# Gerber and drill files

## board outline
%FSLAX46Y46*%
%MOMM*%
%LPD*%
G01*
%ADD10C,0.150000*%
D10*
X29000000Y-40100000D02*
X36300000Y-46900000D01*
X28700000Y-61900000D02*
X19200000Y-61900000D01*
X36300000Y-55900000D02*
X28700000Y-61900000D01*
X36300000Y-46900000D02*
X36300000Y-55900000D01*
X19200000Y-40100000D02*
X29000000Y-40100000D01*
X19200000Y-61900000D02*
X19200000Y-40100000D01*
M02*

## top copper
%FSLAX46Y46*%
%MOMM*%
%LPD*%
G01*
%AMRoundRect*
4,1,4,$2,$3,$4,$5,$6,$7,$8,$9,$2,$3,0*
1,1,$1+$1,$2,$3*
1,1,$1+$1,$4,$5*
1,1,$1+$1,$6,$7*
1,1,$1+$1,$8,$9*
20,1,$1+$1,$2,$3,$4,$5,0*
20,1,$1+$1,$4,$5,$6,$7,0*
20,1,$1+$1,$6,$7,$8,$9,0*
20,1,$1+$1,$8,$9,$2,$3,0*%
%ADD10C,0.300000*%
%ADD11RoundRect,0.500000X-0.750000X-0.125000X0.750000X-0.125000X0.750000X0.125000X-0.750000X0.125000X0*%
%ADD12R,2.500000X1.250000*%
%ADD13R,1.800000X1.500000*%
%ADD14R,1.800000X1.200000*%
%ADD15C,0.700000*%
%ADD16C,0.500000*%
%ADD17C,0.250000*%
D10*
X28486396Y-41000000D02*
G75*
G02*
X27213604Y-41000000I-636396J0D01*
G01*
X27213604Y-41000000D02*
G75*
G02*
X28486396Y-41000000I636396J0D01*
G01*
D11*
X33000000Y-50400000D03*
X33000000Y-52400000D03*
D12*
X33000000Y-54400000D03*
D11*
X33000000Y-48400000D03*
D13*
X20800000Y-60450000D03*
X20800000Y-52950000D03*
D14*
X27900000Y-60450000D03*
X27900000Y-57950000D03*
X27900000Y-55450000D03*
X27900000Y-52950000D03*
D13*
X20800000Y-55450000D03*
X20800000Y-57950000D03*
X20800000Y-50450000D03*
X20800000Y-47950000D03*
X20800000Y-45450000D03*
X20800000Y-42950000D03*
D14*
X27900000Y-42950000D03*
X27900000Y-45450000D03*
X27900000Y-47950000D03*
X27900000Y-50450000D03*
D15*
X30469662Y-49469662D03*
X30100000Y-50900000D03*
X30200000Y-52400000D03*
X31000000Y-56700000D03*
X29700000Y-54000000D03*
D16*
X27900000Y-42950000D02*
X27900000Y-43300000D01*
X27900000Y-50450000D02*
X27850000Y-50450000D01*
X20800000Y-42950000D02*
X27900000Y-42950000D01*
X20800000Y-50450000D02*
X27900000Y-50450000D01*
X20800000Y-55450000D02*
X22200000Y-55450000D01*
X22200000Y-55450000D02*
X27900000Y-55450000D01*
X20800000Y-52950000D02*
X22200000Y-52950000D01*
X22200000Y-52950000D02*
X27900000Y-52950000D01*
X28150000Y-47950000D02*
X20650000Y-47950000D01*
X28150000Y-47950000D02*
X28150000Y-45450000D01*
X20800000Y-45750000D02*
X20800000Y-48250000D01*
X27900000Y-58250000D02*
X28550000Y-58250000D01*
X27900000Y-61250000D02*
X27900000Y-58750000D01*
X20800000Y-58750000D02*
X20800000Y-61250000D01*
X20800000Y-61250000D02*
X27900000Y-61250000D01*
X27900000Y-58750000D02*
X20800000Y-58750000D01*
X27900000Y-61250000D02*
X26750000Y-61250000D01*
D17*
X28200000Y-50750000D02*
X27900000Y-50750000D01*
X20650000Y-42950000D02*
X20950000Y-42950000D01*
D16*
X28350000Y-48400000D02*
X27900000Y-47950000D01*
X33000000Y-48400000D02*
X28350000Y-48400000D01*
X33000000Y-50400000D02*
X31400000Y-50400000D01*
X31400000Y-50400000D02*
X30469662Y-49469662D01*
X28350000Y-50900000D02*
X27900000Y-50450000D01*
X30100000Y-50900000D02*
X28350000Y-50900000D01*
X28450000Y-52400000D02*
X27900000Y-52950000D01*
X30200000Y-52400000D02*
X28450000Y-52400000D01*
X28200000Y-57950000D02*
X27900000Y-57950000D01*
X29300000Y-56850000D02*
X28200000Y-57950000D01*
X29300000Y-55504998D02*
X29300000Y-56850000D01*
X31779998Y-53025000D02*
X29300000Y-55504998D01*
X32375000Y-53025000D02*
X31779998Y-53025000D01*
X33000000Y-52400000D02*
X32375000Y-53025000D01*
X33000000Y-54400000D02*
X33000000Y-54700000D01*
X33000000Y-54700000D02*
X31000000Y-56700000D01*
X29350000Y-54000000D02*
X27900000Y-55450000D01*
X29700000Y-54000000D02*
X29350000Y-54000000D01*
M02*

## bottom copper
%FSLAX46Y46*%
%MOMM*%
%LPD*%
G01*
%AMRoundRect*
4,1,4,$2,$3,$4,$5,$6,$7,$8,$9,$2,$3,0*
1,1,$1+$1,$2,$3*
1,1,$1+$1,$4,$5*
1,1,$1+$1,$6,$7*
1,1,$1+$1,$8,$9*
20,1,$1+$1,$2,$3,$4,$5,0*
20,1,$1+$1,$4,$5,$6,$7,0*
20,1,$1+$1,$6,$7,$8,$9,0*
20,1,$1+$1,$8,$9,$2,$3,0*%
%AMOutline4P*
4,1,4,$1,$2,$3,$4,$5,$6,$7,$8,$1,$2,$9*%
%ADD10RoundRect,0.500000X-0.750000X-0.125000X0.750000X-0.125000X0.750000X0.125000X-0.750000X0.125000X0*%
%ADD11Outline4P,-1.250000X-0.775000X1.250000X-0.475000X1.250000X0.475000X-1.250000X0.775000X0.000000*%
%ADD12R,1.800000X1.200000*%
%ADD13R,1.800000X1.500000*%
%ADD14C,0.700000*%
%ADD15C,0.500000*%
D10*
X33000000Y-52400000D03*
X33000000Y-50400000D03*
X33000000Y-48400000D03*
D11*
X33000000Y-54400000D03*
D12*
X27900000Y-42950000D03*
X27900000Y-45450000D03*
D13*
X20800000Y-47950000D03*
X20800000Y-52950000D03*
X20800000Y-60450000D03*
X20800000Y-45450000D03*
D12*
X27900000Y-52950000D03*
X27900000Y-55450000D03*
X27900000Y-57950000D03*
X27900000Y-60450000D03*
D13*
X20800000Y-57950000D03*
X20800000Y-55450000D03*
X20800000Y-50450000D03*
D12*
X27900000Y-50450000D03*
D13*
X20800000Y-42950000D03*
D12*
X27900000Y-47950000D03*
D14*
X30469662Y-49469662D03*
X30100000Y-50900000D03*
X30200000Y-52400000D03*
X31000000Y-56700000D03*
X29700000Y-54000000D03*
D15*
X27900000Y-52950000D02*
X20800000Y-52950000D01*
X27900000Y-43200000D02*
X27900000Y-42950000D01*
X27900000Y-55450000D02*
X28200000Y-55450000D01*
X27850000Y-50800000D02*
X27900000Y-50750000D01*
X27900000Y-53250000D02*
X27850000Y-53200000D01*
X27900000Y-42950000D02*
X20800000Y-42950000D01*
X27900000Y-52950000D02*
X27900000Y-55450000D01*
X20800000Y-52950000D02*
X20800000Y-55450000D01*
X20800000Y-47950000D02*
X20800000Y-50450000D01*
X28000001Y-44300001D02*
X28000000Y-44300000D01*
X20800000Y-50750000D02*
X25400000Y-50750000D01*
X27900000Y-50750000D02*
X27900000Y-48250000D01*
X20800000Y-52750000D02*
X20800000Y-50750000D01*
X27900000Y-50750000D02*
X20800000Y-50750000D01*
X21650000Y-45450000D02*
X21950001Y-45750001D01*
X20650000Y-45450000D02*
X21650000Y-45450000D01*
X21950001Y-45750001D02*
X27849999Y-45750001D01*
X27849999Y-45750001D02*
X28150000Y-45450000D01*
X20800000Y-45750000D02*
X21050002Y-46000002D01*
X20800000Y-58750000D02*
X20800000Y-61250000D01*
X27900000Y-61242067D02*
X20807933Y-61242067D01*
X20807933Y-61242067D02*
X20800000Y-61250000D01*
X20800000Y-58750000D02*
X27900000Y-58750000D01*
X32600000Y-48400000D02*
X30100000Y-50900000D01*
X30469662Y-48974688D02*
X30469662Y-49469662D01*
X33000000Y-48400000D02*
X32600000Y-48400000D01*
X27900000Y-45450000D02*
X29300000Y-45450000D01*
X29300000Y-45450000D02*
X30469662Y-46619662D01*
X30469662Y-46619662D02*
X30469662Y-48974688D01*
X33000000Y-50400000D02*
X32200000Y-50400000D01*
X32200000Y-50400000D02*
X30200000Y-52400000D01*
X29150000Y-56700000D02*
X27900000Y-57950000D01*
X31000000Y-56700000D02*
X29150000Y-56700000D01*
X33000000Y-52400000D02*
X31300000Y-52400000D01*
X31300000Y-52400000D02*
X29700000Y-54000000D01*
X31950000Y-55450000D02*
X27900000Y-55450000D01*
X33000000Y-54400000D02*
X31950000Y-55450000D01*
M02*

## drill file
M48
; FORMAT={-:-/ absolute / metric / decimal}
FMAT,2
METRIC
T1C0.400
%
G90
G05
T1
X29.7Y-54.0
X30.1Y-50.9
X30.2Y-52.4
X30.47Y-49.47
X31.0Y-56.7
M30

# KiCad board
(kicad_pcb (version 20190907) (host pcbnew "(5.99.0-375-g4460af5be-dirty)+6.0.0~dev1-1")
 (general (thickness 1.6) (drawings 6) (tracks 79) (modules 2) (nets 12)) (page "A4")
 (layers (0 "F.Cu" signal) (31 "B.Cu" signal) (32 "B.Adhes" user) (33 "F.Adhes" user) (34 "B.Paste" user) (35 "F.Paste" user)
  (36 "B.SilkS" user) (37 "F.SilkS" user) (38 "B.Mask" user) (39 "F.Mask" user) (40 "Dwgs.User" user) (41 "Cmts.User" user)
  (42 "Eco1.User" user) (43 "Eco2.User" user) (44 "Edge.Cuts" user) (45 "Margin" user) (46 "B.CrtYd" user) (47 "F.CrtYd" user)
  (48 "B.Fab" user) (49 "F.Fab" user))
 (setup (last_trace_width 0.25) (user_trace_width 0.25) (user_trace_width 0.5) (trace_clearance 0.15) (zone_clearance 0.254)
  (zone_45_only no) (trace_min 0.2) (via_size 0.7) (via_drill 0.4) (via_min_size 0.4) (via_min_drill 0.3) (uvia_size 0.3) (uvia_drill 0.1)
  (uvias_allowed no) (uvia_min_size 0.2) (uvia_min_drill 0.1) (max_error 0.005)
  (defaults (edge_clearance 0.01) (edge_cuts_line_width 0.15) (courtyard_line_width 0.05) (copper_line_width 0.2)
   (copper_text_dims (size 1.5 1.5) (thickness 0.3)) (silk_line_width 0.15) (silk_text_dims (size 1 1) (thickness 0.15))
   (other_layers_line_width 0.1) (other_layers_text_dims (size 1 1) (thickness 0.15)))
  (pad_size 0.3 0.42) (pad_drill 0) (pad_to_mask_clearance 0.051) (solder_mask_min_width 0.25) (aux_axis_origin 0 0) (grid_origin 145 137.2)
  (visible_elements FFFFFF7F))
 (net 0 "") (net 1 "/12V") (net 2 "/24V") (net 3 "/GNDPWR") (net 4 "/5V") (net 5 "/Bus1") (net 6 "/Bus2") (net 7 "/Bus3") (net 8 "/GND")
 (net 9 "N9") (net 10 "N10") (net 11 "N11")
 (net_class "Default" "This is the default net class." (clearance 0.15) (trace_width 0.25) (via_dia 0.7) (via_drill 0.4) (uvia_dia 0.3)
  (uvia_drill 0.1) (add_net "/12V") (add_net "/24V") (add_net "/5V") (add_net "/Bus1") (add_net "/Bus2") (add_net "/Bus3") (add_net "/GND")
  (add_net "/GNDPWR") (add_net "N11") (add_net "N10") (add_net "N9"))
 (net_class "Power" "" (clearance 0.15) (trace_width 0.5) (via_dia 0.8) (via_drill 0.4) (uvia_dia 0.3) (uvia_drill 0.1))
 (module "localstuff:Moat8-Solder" (layer "B.Cu") (at 33 55.9)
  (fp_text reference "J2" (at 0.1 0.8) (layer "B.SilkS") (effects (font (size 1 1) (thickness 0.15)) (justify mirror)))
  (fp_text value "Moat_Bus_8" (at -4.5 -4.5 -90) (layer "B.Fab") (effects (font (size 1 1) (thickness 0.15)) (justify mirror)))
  (pad "6" smd roundrect (at 0 -5.5) (size 2.5 1.25) (layers "F.Cu" "F.Mask") (roundrect_rratio 0.4) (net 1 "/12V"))
  (pad "7" smd roundrect (at 0 -3.5) (size 2.5 1.25) (layers "F.Cu" "F.Mask") (roundrect_rratio 0.4) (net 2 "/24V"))
  (pad "8" smd rect (at 0 -1.5) (size 2.5 1.25) (layers "F.Cu" "F.Mask") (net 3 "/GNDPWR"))
  (pad "5" smd roundrect (at 0 -7.5) (size 2.5 1.25) (layers "F.Cu" "F.Mask") (roundrect_rratio 0.4) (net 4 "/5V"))
  (pad "2" smd roundrect (at 0 -3.5) (size 2.5 1.25) (layers "B.Cu" "B.Mask") (roundrect_rratio 0.4) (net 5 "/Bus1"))
  (pad "3" smd roundrect (at 0 -5.5) (size 2.5 1.25) (layers "B.Cu" "B.Mask") (roundrect_rratio 0.4) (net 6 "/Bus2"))
  (pad "4" smd roundrect (at 0 -7.5) (size 2.5 1.25) (layers "B.Cu" "B.Mask") (roundrect_rratio 0.4) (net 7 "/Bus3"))
  (pad "1" smd trapezoid (at 0 -1.5) (size 2.5 1.25) (rect_delta 0.3 0) (layers "B.Cu" "B.Mask") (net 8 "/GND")))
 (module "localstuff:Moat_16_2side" (layer "F.Cu") (at 24.4 52 -90)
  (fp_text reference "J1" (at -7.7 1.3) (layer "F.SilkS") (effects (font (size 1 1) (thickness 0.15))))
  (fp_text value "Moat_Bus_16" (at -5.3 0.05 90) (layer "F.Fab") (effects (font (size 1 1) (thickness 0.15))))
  (fp_circle (center -11 -3.45) (end -10.363604 -3.45) (layer "F.Cu") (width 0.3))
  (pad "2" smd rect (at -9.05 -3.5 90) (size 1.2 1.8) (layers "B.Cu" "B.Paste" "B.Mask") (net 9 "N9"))
  (pad "4" smd rect (at -6.55 -3.5 90) (size 1.2 1.8) (layers "B.Cu" "B.Paste" "B.Mask") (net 1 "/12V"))
  (pad "6" smd rect (at -4.05 3.6 90) (size 1.5 1.8) (layers "B.Cu" "B.Paste" "B.Mask") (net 8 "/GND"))
  (pad "10" smd rect (at 0.95 3.6 90) (size 1.5 1.8) (layers "B.Cu" "B.Paste" "B.Mask") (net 8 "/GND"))
  (pad "16" smd rect (at 8.45 3.6 90) (size 1.5 1.8) (layers "B.Cu" "B.Paste" "B.Mask") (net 3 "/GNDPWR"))
  (pad "4" smd rect (at -6.55 3.6 90) (size 1.5 1.8) (layers "B.Cu" "B.Paste" "B.Mask") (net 1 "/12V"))
  (pad "10" smd rect (at 0.95 -3.5 90) (size 1.2 1.8) (layers "B.Cu" "B.Paste" "B.Mask") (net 8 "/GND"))
  (pad "12" smd rect (at 3.45 -3.5 90) (size 1.2 1.8) (layers "B.Cu" "B.Paste" "B.Mask") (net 8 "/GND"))
  (pad "14" smd rect (at 5.95 -3.5 90) (size 1.2 1.8) (layers "B.Cu" "B.Paste" "B.Mask") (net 3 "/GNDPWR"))
  (pad "16" smd rect (at 8.45 -3.5 90) (size 1.2 1.8) (layers "B.Cu" "B.Paste" "B.Mask") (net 3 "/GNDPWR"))
  (pad "14" smd rect (at 5.95 3.6 90) (size 1.5 1.8) (layers "B.Cu" "B.Paste" "B.Mask") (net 3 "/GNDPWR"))
  (pad "12" smd rect (at 3.45 3.6 90) (size 1.5 1.8) (layers "B.Cu" "B.Paste" "B.Mask") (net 8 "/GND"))
  (pad "8" smd rect (at -1.55 3.6 90) (size 1.5 1.8) (layers "B.Cu" "B.Paste" "B.Mask") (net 8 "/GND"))
  (pad "8" smd rect (at -1.55 -3.5 90) (size 1.2 1.8) (layers "B.Cu" "B.Paste" "B.Mask") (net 8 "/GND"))
  (pad "2" smd rect (at -9.05 3.6 90) (size 1.5 1.8) (layers "B.Cu" "B.Paste" "B.Mask") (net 9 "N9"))
  (pad "6" smd rect (at -4.05 -3.5 90) (size 1.2 1.8) (layers "B.Cu" "B.Paste" "B.Mask") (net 8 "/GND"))
  (pad "15" smd rect (at 8.45 3.6 270) (size 1.5 1.8) (layers "F.Cu" "F.Paste" "F.Mask") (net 2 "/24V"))
  (pad "9" smd rect (at 0.95 3.6 270) (size 1.5 1.8) (layers "F.Cu" "F.Paste" "F.Mask") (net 6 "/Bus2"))
  (pad "15" smd rect (at 8.45 -3.5 270) (size 1.2 1.8) (layers "F.Cu" "F.Paste" "F.Mask") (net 2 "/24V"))
  (pad "13" smd rect (at 5.95 -3.5 270) (size 1.2 1.8) (layers "F.Cu" "F.Paste" "F.Mask") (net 2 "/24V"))
  (pad "11" smd rect (at 3.45 -3.5 270) (size 1.2 1.8) (layers "F.Cu" "F.Paste" "F.Mask") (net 5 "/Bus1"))
  (pad "9" smd rect (at 0.95 -3.5 270) (size 1.2 1.8) (layers "F.Cu" "F.Paste" "F.Mask") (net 6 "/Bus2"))
  (pad "11" smd rect (at 3.45 3.6 270) (size 1.5 1.8) (layers "F.Cu" "F.Paste" "F.Mask") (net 5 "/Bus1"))
  (pad "13" smd rect (at 5.95 3.6 270) (size 1.5 1.8) (layers "F.Cu" "F.Paste" "F.Mask") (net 2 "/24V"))
  (pad "7" smd rect (at -1.55 3.6 270) (size 1.5 1.8) (layers "F.Cu" "F.Paste" "F.Mask") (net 7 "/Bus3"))
  (pad "5" smd rect (at -4.05 3.6 270) (size 1.5 1.8) (layers "F.Cu" "F.Paste" "F.Mask") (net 4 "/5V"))
  (pad "3" smd rect (at -6.55 3.6 270) (size 1.5 1.8) (layers "F.Cu" "F.Paste" "F.Mask") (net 4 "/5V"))
  (pad "1" smd rect (at -9.05 3.6 270) (size 1.5 1.8) (layers "F.Cu" "F.Paste" "F.Mask") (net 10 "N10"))
  (pad "1" smd rect (at -9.05 -3.5 270) (size 1.2 1.8) (layers "F.Cu" "F.Paste" "F.Mask") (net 10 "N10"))
  (pad "3" smd rect (at -6.55 -3.5 270) (size 1.2 1.8) (layers "F.Cu" "F.Paste" "F.Mask") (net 4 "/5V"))
  (pad "5" smd rect (at -4.05 -3.5 270) (size 1.2 1.8) (layers "F.Cu" "F.Paste" "F.Mask") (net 4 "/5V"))
  (pad "7" smd rect (at -1.55 -3.5 270) (size 1.2 1.8) (layers "F.Cu" "F.Paste" "F.Mask") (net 7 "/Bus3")))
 (gr_line (start 29 40.1) (end 36.3 46.9) (layer "Edge.Cuts") (width 0.15))
 (gr_line (start 28.7 61.9) (end 19.2 61.9) (layer "Edge.Cuts") (width 0.15))
 (gr_line (start 36.3 55.9) (end 28.7 61.9) (layer "Edge.Cuts") (width 0.15))
 (gr_line (start 36.3 46.9) (end 36.3 55.9) (layer "Edge.Cuts") (width 0.15))
 (gr_line (start 19.2 40.1) (end 29 40.1) (layer "Edge.Cuts") (width 0.15))
 (gr_line (start 19.2 61.9) (end 19.2 40.1) (layer "Edge.Cuts") (width 0.15))
 (segment (start 27.9 52.95) (end 20.8 52.95) (width 0.5) (layer "B.Cu") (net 8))
 (segment (start 27.9 42.95) (end 27.9 43.3) (width 0.5) (layer "F.Cu") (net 10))
 (segment (start 27.9 43.2) (end 27.9 42.95) (width 0.5) (layer "B.Cu") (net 9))
 (segment (start 27.9 55.45) (end 28.2 55.45) (width 0.5) (layer "B.Cu") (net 8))
 (segment (start 27.85 50.8) (end 27.9 50.75) (width 0.5) (layer "B.Cu") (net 8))
 (segment (start 27.9 53.25) (end 27.85 53.2) (width 0.5) (layer "B.Cu") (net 8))
 (segment (start 27.9 50.45) (end 27.85 50.45) (width 0.5) (layer "F.Cu") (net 7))
 (segment (start 20.8 42.95) (end 27.9 42.95) (width 0.5) (layer "F.Cu") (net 10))
 (segment (start 27.9 42.95) (end 20.8 42.95) (width 0.5) (layer "B.Cu") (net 9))
 (segment (start 20.8 50.45) (end 27.9 50.45) (width 0.5) (layer "F.Cu") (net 7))
 (segment (start 20.8 55.45) (end 22.2 55.45) (width 0.5) (layer "F.Cu") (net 5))
 (segment (start 22.2 55.45) (end 27.9 55.45) (width 0.5) (layer "F.Cu") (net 5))
 (segment (start 20.8 52.95) (end 22.2 52.95) (width 0.5) (layer "F.Cu") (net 6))
 (segment (start 22.2 52.95) (end 27.9 52.95) (width 0.5) (layer "F.Cu") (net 6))
 (segment (start 27.9 52.95) (end 27.9 55.45) (width 0.5) (layer "B.Cu") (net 8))
 (segment (start 20.8 52.95) (end 20.8 55.45) (width 0.5) (layer "B.Cu") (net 8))
 (segment (start 20.8 47.95) (end 20.8 50.45) (width 0.5) (layer "B.Cu") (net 8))
 (segment (start 28.15 47.95) (end 20.65 47.95) (width 0.5) (layer "F.Cu") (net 4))
 (segment (start 28.15 47.95) (end 28.15 45.45) (width 0.5) (layer "F.Cu") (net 4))
 (segment (start 28.000001 44.300001) (end 28 44.3) (width 0.5) (layer "B.Cu") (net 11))
 (segment (start 20.8 45.75) (end 20.8 48.25) (width 0.5) (layer "F.Cu") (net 4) (status 30))
 (segment (start 27.9 58.25) (end 28.55 58.25) (width 0.5) (layer "F.Cu") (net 2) (status 30))
 (segment (start 27.9 61.25) (end 27.9 58.75) (width 0.5) (layer "F.Cu") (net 2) (status 30))
 (segment (start 20.8 58.75) (end 20.8 61.25) (width 0.5) (layer "F.Cu") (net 2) (status 30))
 (segment (start 20.8 61.25) (end 27.9 61.25) (width 0.5) (layer "F.Cu") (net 2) (status 30))
 (segment (start 27.9 58.75) (end 20.8 58.75) (width 0.5) (layer "F.Cu") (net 2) (status 30))
 (segment (start 27.9 61.25) (end 26.75 61.25) (width 0.5) (layer "F.Cu") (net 2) (status 10))
 (segment (start 20.8 50.75) (end 25.4 50.75) (width 0.5) (layer "B.Cu") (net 8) (status 10))
 (segment (start 27.9 50.75) (end 27.9 48.25) (width 0.5) (layer "B.Cu") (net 8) (status 30))
 (segment (start 20.8 52.75) (end 20.8 50.75) (width 0.5) (layer "B.Cu") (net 8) (status 30))
 (segment (start 27.9 50.75) (end 20.8 50.75) (width 0.5) (layer "B.Cu") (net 8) (status 30))
 (segment (start 21.65 45.45) (end 21.950001 45.750001) (width 0.5) (layer "B.Cu") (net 1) (status 10))
 (segment (start 20.65 45.45) (end 21.65 45.45) (width 0.5) (layer "B.Cu") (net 1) (status 30))
 (segment (start 21.950001 45.750001) (end 27.849999 45.750001) (width 0.5) (layer "B.Cu") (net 1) (status 20))
 (segment (start 27.849999 45.750001) (end 28.15 45.45) (width 0.5) (layer "B.Cu") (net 1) (status 30))
 (segment (start 20.8 45.75) (end 21.050002 46.000002) (width 0.5) (layer "B.Cu") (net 1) (status 30))
 (segment (start 20.8 58.75) (end 20.8 61.25) (width 0.5) (layer "B.Cu") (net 3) (status 30))
 (segment (start 27.9 61.242067) (end 20.807933 61.242067) (width 0.5) (layer "B.Cu") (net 3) (status 30))
 (segment (start 20.807933 61.242067) (end 20.8 61.25) (width 0.5) (layer "B.Cu") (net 3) (status 30))
 (segment (start 20.8 58.75) (end 27.9 58.75) (width 0.5) (layer "B.Cu") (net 3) (status 30))
 (segment (start 28.2 50.75) (end 27.9 50.75) (width 0.25) (layer "F.Cu") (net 7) (status 30))
 (segment (start 20.65 42.95) (end 20.95 42.95) (width 0.25) (layer "F.Cu") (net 10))
 (segment (start 28.35 48.4) (end 27.9 47.95) (width 0.5) (layer "F.Cu") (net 4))
 (segment (start 33 48.4) (end 28.35 48.4) (width 0.5) (layer "F.Cu") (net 4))
 (segment (start 32.6 48.4) (end 30.1 50.9) (width 0.5) (layer "B.Cu") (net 7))
 (via (at 30.469662 49.469662) (size 0.7) (drill 0.4) (layers "F.Cu" "B.Cu") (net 1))
 (segment (start 30.469662 48.974688) (end 30.469662 49.469662) (width 0.5) (layer "B.Cu") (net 1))
 (segment (start 33 48.4) (end 32.6 48.4) (width 0.5) (layer "B.Cu") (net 7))
 (segment (start 27.9 45.45) (end 29.3 45.45) (width 0.5) (layer "B.Cu") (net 1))
 (via (at 30.1 50.9) (size 0.7) (drill 0.4) (layers "F.Cu" "B.Cu") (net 7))
 (segment (start 29.3 45.45) (end 30.469662 46.619662) (width 0.5) (layer "B.Cu") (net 1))
 (segment (start 33 50.4) (end 31.4 50.4) (width 0.5) (layer "F.Cu") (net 1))
 (segment (start 30.469662 46.619662) (end 30.469662 48.974688) (width 0.5) (layer "B.Cu") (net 1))
 (segment (start 31.4 50.4) (end 30.469662 49.469662) (width 0.5) (layer "F.Cu") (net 1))
 (segment (start 28.35 50.9) (end 27.9 50.45) (width 0.5) (layer "F.Cu") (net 7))
 (segment (start 30.1 50.9) (end 28.35 50.9) (width 0.5) (layer "F.Cu") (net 7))
 (via (at 30.2 52.4) (size 0.7) (drill 0.4) (layers "F.Cu" "B.Cu") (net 6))
 (segment (start 33 50.4) (end 32.2 50.4) (width 0.5) (layer "B.Cu") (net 6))
 (segment (start 32.2 50.4) (end 30.2 52.4) (width 0.5) (layer "B.Cu") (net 6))
 (segment (start 28.45 52.4) (end 27.9 52.95) (width 0.5) (layer "F.Cu") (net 6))
 (segment (start 30.2 52.4) (end 28.45 52.4) (width 0.5) (layer "F.Cu") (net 6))
 (segment (start 28.2 57.95) (end 27.9 57.95) (width 0.5) (layer "F.Cu") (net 2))
 (segment (start 29.3 56.85) (end 28.2 57.95) (width 0.5) (layer "F.Cu") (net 2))
 (segment (start 29.3 55.504998) (end 29.3 56.85) (width 0.5) (layer "F.Cu") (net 2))
 (segment (start 31.779998 53.025) (end 29.3 55.504998) (width 0.5) (layer "F.Cu") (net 2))
 (segment (start 32.375 53.025) (end 31.779998 53.025) (width 0.5) (layer "F.Cu") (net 2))
 (segment (start 33 52.4) (end 32.375 53.025) (width 0.5) (layer "F.Cu") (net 2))
 (via (at 31 56.7) (size 0.7) (drill 0.4) (layers "F.Cu" "B.Cu") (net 3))
 (segment (start 33 54.4) (end 33 54.7) (width 0.5) (layer "F.Cu") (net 3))
 (segment (start 33 54.7) (end 31 56.7) (width 0.5) (layer "F.Cu") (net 3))
 (segment (start 29.15 56.7) (end 27.9 57.95) (width 0.5) (layer "B.Cu") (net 3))
 (segment (start 31 56.7) (end 29.15 56.7) (width 0.5) (layer "B.Cu") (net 3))
 (via (at 29.7 54) (size 0.7) (drill 0.4) (layers "F.Cu" "B.Cu") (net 5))
 (segment (start 33 52.4) (end 31.3 52.4) (width 0.5) (layer "B.Cu") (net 5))
 (segment (start 31.3 52.4) (end 29.7 54) (width 0.5) (layer "B.Cu") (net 5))
 (segment (start 29.35 54) (end 27.9 55.45) (width 0.5) (layer "F.Cu") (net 5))
 (segment (start 29.7 54) (end 29.35 54) (width 0.5) (layer "F.Cu") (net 5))
 (segment (start 31.95 55.45) (end 27.9 55.45) (width 0.5) (layer "B.Cu") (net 8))
 (segment (start 33 54.4) (end 31.95 55.45) (width 0.5) (layer "B.Cu") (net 8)))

